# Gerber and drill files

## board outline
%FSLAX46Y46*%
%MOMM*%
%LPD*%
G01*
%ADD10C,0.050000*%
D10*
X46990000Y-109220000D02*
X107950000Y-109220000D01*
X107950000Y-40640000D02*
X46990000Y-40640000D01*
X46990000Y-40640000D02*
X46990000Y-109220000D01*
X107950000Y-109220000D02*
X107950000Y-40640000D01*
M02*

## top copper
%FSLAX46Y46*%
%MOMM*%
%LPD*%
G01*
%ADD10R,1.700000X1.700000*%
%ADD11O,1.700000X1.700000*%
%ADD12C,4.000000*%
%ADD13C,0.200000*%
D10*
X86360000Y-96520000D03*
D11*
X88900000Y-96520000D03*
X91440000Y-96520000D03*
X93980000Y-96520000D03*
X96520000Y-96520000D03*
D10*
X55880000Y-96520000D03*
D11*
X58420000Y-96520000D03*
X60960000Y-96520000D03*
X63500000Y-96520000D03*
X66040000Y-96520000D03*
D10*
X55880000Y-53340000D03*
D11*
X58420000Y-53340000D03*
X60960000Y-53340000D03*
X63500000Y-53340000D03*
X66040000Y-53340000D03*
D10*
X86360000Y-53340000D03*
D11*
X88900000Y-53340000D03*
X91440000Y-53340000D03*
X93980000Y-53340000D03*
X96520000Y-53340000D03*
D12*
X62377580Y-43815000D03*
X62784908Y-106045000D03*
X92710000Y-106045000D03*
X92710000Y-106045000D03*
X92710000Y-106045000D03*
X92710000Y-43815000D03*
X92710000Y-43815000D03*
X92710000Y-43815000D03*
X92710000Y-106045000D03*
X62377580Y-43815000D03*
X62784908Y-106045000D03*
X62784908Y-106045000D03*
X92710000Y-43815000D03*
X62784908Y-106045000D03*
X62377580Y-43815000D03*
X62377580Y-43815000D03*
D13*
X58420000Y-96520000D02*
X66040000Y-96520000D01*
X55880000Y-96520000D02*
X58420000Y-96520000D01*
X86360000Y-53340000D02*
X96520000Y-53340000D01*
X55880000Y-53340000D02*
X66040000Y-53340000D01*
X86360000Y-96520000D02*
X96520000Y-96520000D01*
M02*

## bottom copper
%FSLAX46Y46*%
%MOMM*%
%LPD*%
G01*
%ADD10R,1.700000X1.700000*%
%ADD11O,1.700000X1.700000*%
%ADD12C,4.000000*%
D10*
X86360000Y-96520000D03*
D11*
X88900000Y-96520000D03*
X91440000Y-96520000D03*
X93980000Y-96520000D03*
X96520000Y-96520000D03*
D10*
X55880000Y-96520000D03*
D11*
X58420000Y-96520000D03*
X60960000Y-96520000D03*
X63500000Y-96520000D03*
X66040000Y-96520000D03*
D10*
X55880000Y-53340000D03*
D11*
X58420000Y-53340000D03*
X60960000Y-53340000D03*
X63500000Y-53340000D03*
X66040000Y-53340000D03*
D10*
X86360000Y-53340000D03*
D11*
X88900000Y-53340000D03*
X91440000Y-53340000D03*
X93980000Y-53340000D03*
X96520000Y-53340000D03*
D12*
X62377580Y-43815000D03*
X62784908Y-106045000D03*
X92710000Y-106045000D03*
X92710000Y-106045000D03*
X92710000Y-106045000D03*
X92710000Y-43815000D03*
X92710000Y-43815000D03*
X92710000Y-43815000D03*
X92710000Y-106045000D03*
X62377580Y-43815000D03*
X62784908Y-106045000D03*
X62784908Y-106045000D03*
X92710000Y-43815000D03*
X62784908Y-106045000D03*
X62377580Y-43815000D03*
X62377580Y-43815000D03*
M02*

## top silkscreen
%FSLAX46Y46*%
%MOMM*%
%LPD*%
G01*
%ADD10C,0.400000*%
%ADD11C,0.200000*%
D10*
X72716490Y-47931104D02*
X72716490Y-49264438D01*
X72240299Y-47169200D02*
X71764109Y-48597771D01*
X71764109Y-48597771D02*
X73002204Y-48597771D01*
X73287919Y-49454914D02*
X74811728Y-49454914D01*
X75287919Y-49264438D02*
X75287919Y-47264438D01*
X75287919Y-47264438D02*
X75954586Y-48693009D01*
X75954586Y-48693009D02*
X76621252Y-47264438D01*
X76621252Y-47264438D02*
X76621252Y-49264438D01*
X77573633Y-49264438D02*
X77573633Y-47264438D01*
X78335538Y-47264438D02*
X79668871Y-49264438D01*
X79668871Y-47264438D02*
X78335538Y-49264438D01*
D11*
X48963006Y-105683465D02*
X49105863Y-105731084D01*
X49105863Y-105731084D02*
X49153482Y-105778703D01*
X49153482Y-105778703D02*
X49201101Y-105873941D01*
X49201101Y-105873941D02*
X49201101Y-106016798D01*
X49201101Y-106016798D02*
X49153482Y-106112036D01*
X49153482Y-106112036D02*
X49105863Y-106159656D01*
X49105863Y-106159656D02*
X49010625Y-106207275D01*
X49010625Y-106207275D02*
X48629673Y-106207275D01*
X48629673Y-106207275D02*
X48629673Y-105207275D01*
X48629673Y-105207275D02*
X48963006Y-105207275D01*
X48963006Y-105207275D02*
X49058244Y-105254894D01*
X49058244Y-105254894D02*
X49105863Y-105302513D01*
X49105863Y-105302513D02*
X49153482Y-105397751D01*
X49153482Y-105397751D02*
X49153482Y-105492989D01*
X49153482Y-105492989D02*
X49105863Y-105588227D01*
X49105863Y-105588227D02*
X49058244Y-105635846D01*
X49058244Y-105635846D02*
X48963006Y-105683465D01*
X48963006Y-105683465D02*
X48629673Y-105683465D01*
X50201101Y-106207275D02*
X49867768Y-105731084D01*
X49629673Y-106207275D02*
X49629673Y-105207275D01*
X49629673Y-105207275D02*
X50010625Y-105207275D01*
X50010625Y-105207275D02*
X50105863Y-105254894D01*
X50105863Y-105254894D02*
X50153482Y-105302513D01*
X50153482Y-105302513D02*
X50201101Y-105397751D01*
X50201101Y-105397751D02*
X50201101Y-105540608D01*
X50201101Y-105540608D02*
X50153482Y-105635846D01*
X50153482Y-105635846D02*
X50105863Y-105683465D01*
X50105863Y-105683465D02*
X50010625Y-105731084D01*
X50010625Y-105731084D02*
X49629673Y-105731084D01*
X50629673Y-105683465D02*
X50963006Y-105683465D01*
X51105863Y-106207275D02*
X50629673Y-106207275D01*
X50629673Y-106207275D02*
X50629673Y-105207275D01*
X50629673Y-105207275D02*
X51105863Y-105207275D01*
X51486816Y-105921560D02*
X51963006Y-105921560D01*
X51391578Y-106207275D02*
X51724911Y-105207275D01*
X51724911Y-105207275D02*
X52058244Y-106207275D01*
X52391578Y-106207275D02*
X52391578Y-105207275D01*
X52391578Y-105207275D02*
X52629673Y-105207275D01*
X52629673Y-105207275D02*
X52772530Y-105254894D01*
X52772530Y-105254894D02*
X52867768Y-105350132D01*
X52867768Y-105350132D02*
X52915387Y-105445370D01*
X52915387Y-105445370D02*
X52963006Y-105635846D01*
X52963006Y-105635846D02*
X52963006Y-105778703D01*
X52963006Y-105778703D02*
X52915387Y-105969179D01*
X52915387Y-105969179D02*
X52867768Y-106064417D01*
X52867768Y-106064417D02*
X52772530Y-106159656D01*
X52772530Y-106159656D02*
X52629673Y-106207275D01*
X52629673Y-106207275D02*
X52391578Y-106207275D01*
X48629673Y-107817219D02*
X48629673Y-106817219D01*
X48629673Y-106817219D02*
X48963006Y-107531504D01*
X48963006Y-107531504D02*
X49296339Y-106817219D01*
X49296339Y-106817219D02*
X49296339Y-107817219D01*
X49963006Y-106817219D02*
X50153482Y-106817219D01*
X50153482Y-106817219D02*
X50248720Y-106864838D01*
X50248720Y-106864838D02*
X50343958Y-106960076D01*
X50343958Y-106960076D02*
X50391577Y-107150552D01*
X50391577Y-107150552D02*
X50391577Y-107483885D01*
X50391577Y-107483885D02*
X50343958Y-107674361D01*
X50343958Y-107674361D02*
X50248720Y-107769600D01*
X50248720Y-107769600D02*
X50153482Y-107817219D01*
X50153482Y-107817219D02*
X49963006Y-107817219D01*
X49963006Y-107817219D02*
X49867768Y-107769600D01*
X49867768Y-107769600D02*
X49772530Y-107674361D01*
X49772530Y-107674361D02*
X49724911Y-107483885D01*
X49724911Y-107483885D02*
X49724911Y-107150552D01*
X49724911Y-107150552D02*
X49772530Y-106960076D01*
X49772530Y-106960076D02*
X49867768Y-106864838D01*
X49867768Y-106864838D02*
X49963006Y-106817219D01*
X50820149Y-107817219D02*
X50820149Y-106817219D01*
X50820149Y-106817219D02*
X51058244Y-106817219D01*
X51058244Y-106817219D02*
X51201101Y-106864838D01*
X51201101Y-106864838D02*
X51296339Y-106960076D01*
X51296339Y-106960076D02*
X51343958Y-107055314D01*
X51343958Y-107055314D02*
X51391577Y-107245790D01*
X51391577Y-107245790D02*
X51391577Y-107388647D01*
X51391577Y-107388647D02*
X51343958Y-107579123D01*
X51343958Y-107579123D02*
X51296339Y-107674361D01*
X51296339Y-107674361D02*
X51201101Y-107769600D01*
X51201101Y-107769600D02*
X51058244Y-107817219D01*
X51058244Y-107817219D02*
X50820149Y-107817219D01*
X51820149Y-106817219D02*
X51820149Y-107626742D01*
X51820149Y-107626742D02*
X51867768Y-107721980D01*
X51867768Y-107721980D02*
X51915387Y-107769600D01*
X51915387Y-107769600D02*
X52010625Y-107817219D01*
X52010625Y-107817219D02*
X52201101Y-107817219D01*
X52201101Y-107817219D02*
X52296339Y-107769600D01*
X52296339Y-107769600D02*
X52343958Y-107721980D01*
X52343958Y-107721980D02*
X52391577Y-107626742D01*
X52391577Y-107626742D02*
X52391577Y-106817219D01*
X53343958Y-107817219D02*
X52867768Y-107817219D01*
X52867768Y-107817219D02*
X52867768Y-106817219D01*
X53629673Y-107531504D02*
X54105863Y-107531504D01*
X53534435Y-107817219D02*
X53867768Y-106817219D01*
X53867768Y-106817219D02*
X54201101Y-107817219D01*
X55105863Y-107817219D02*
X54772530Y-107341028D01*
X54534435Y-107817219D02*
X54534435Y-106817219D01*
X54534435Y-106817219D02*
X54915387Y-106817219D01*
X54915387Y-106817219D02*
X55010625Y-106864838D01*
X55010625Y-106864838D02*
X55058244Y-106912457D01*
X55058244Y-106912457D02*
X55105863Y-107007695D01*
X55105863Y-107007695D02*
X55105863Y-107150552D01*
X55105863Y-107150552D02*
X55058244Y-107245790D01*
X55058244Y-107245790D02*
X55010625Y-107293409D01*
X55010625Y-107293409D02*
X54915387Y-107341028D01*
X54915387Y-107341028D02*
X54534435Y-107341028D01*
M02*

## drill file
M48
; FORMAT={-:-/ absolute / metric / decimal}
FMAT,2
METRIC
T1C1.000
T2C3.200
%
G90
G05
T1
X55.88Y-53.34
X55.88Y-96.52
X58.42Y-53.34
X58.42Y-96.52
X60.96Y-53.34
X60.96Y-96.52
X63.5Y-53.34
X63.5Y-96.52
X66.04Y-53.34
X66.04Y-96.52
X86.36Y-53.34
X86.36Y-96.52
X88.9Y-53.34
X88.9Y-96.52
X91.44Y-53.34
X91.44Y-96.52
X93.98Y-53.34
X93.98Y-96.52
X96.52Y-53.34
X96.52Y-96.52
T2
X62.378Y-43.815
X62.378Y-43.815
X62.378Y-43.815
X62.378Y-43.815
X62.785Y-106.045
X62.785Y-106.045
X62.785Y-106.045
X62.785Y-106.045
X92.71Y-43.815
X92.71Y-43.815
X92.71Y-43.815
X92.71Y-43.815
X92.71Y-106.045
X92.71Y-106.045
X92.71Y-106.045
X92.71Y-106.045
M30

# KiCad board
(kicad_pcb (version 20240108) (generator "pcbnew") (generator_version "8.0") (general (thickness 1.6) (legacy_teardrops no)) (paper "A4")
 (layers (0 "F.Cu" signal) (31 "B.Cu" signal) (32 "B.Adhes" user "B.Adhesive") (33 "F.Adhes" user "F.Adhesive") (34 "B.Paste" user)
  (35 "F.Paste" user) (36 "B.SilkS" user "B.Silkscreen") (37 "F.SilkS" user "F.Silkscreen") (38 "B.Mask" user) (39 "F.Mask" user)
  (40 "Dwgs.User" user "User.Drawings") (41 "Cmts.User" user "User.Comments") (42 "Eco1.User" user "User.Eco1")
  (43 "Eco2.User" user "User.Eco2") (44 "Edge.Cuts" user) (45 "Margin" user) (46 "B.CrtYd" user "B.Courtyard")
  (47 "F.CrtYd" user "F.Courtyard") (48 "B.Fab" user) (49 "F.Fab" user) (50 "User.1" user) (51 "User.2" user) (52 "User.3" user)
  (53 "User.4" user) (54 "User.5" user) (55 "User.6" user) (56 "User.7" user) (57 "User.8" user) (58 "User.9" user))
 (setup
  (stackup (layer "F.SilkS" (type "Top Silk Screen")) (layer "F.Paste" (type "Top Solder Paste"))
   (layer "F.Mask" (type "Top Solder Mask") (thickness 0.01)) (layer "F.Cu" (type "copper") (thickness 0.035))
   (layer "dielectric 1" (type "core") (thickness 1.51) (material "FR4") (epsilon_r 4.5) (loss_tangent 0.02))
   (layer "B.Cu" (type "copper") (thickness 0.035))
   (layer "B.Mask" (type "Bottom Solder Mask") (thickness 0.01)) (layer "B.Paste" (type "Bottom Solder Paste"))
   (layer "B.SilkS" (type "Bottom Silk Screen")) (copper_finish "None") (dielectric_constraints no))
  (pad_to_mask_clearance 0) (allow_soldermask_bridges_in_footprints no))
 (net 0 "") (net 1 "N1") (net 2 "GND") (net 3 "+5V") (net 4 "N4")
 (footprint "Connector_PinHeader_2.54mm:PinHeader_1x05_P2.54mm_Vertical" (layer "B.Cu") (at 86.36 96.52 -90)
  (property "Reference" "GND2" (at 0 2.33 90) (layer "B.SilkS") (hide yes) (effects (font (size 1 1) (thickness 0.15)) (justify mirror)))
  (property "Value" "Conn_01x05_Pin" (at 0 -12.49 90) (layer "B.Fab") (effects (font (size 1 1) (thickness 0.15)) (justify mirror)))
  (pad "1" thru_hole rect (at 0 0 270) (size 1.7 1.7) (drill 1) (layers "*.Cu" "*.Mask") (remove_unused_layers no) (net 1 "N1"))
  (pad "2" thru_hole oval (at 0 -2.54 270) (size 1.7 1.7) (drill 1) (layers "*.Cu" "*.Mask") (remove_unused_layers no) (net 1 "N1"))
  (pad "3" thru_hole oval (at 0 -5.08 270) (size 1.7 1.7) (drill 1) (layers "*.Cu" "*.Mask") (remove_unused_layers no) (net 1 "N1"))
  (pad "4" thru_hole oval (at 0 -7.62 270) (size 1.7 1.7) (drill 1) (layers "*.Cu" "*.Mask") (remove_unused_layers no) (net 1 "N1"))
  (pad "5" thru_hole oval (at 0 -10.16 270) (size 1.7 1.7) (drill 1) (layers "*.Cu" "*.Mask") (remove_unused_layers no) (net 1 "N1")))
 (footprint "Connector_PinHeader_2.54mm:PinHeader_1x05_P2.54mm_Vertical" (layer "B.Cu") (at 55.88 96.52 -90)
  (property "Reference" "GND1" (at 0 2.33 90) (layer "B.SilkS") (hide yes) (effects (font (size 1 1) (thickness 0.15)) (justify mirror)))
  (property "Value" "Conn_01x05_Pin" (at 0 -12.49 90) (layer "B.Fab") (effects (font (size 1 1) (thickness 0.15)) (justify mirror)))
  (pad "1" thru_hole rect (at 0 0 270) (size 1.7 1.7) (drill 1) (layers "*.Cu" "*.Mask") (remove_unused_layers no) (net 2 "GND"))
  (pad "2" thru_hole oval (at 0 -2.54 270) (size 1.7 1.7) (drill 1) (layers "*.Cu" "*.Mask") (remove_unused_layers no) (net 2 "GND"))
  (pad "3" thru_hole oval (at 0 -5.08 270) (size 1.7 1.7) (drill 1) (layers "*.Cu" "*.Mask") (remove_unused_layers no) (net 2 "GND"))
  (pad "4" thru_hole oval (at 0 -7.62 270) (size 1.7 1.7) (drill 1) (layers "*.Cu" "*.Mask") (remove_unused_layers no) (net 2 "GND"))
  (pad "5" thru_hole oval (at 0 -10.16 270) (size 1.7 1.7) (drill 1) (layers "*.Cu" "*.Mask") (remove_unused_layers no) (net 2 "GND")))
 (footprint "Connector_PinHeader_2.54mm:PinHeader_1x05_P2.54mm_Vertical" (layer "B.Cu") (at 55.88 53.34 -90)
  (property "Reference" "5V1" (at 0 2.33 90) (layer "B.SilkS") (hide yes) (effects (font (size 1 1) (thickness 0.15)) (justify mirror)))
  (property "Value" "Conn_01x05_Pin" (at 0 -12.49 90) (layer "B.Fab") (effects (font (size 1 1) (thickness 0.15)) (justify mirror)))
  (pad "1" thru_hole rect (at 0 0 270) (size 1.7 1.7) (drill 1) (layers "*.Cu" "*.Mask") (remove_unused_layers no) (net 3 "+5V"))
  (pad "2" thru_hole oval (at 0 -2.54 270) (size 1.7 1.7) (drill 1) (layers "*.Cu" "*.Mask") (remove_unused_layers no) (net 3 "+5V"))
  (pad "3" thru_hole oval (at 0 -5.08 270) (size 1.7 1.7) (drill 1) (layers "*.Cu" "*.Mask") (remove_unused_layers no) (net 3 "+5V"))
  (pad "4" thru_hole oval (at 0 -7.62 270) (size 1.7 1.7) (drill 1) (layers "*.Cu" "*.Mask") (remove_unused_layers no) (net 3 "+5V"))
  (pad "5" thru_hole oval (at 0 -10.16 270) (size 1.7 1.7) (drill 1) (layers "*.Cu" "*.Mask") (remove_unused_layers no) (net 3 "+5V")))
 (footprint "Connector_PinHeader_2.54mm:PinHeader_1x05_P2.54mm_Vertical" (layer "B.Cu") (at 86.36 53.34 -90)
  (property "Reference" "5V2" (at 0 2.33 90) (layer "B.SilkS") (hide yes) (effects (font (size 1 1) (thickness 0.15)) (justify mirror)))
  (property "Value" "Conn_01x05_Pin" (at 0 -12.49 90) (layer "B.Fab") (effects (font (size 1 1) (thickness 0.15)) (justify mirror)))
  (pad "1" thru_hole rect (at 0 0 270) (size 1.7 1.7) (drill 1) (layers "*.Cu" "*.Mask") (remove_unused_layers no) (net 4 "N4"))
  (pad "2" thru_hole oval (at 0 -2.54 270) (size 1.7 1.7) (drill 1) (layers "*.Cu" "*.Mask") (remove_unused_layers no) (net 4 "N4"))
  (pad "3" thru_hole oval (at 0 -5.08 270) (size 1.7 1.7) (drill 1) (layers "*.Cu" "*.Mask") (remove_unused_layers no) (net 4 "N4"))
  (pad "4" thru_hole oval (at 0 -7.62 270) (size 1.7 1.7) (drill 1) (layers "*.Cu" "*.Mask") (remove_unused_layers no) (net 4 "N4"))
  (pad "5" thru_hole oval (at 0 -10.16 270) (size 1.7 1.7) (drill 1) (layers "*.Cu" "*.Mask") (remove_unused_layers no) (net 4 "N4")))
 (gr_line (start 46.99 109.22) (end 107.95 109.22) (stroke (width 0.05) (type default)) (layer "Edge.Cuts"))
 (gr_line (start 107.95 40.64) (end 46.99 40.64) (stroke (width 0.05) (type default)) (layer "Edge.Cuts"))
 (gr_line (start 46.99 40.64) (end 46.99 109.22) (stroke (width 0.05) (type default)) (layer "Edge.Cuts"))
 (gr_line (start 107.95 109.22) (end 107.95 40.64) (stroke (width 0.05) (type default)) (layer "Edge.Cuts"))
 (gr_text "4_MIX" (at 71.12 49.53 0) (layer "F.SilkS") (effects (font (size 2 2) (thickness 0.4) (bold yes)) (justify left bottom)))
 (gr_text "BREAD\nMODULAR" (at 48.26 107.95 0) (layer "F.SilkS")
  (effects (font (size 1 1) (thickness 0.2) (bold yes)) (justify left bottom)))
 (via (at 62.37758 43.815) (size 4) (drill 3.2) (layers "F.Cu" "B.Cu") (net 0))
 (via (at 62.784908 106.045) (size 4) (drill 3.2) (layers "F.Cu" "B.Cu") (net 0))
 (via (at 92.71 106.045) (size 4) (drill 3.2) (layers "F.Cu" "B.Cu") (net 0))
 (via (at 92.71 106.045) (size 4) (drill 3.2) (layers "F.Cu" "B.Cu") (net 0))
 (via (at 92.71 106.045) (size 4) (drill 3.2) (layers "F.Cu" "B.Cu") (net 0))
 (via (at 92.71 43.815) (size 4) (drill 3.2) (layers "F.Cu" "B.Cu") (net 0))
 (via (at 92.71 43.815) (size 4) (drill 3.2) (layers "F.Cu" "B.Cu") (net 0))
 (via (at 92.71 43.815) (size 4) (drill 3.2) (layers "F.Cu" "B.Cu") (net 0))
 (via (at 92.71 106.045) (size 4) (drill 3.2) (layers "F.Cu" "B.Cu") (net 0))
 (via (at 62.37758 43.815) (size 4) (drill 3.2) (layers "F.Cu" "B.Cu") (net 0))
 (via (at 62.784908 106.045) (size 4) (drill 3.2) (layers "F.Cu" "B.Cu") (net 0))
 (via (at 62.784908 106.045) (size 4) (drill 3.2) (layers "F.Cu" "B.Cu") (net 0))
 (via (at 92.71 43.815) (size 4) (drill 3.2) (layers "F.Cu" "B.Cu") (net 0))
 (via (at 62.784908 106.045) (size 4) (drill 3.2) (layers "F.Cu" "B.Cu") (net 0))
 (via (at 62.37758 43.815) (size 4) (drill 3.2) (layers "F.Cu" "B.Cu") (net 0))
 (via (at 62.37758 43.815) (size 4) (drill 3.2) (layers "F.Cu" "B.Cu") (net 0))
 (segment (start 58.42 96.52) (end 66.04 96.52) (width 0.2) (layer "F.Cu") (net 2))
 (segment (start 55.88 96.52) (end 58.42 96.52) (width 0.2) (layer "F.Cu") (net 2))
 (segment (start 86.36 53.34) (end 96.52 53.34) (width 0.2) (layer "F.Cu") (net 4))
 (segment (start 55.88 53.34) (end 66.04 53.34) (width 0.2) (layer "F.Cu") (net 3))
 (segment (start 86.36 96.52) (end 96.52 96.52) (width 0.2) (layer "F.Cu") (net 1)))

